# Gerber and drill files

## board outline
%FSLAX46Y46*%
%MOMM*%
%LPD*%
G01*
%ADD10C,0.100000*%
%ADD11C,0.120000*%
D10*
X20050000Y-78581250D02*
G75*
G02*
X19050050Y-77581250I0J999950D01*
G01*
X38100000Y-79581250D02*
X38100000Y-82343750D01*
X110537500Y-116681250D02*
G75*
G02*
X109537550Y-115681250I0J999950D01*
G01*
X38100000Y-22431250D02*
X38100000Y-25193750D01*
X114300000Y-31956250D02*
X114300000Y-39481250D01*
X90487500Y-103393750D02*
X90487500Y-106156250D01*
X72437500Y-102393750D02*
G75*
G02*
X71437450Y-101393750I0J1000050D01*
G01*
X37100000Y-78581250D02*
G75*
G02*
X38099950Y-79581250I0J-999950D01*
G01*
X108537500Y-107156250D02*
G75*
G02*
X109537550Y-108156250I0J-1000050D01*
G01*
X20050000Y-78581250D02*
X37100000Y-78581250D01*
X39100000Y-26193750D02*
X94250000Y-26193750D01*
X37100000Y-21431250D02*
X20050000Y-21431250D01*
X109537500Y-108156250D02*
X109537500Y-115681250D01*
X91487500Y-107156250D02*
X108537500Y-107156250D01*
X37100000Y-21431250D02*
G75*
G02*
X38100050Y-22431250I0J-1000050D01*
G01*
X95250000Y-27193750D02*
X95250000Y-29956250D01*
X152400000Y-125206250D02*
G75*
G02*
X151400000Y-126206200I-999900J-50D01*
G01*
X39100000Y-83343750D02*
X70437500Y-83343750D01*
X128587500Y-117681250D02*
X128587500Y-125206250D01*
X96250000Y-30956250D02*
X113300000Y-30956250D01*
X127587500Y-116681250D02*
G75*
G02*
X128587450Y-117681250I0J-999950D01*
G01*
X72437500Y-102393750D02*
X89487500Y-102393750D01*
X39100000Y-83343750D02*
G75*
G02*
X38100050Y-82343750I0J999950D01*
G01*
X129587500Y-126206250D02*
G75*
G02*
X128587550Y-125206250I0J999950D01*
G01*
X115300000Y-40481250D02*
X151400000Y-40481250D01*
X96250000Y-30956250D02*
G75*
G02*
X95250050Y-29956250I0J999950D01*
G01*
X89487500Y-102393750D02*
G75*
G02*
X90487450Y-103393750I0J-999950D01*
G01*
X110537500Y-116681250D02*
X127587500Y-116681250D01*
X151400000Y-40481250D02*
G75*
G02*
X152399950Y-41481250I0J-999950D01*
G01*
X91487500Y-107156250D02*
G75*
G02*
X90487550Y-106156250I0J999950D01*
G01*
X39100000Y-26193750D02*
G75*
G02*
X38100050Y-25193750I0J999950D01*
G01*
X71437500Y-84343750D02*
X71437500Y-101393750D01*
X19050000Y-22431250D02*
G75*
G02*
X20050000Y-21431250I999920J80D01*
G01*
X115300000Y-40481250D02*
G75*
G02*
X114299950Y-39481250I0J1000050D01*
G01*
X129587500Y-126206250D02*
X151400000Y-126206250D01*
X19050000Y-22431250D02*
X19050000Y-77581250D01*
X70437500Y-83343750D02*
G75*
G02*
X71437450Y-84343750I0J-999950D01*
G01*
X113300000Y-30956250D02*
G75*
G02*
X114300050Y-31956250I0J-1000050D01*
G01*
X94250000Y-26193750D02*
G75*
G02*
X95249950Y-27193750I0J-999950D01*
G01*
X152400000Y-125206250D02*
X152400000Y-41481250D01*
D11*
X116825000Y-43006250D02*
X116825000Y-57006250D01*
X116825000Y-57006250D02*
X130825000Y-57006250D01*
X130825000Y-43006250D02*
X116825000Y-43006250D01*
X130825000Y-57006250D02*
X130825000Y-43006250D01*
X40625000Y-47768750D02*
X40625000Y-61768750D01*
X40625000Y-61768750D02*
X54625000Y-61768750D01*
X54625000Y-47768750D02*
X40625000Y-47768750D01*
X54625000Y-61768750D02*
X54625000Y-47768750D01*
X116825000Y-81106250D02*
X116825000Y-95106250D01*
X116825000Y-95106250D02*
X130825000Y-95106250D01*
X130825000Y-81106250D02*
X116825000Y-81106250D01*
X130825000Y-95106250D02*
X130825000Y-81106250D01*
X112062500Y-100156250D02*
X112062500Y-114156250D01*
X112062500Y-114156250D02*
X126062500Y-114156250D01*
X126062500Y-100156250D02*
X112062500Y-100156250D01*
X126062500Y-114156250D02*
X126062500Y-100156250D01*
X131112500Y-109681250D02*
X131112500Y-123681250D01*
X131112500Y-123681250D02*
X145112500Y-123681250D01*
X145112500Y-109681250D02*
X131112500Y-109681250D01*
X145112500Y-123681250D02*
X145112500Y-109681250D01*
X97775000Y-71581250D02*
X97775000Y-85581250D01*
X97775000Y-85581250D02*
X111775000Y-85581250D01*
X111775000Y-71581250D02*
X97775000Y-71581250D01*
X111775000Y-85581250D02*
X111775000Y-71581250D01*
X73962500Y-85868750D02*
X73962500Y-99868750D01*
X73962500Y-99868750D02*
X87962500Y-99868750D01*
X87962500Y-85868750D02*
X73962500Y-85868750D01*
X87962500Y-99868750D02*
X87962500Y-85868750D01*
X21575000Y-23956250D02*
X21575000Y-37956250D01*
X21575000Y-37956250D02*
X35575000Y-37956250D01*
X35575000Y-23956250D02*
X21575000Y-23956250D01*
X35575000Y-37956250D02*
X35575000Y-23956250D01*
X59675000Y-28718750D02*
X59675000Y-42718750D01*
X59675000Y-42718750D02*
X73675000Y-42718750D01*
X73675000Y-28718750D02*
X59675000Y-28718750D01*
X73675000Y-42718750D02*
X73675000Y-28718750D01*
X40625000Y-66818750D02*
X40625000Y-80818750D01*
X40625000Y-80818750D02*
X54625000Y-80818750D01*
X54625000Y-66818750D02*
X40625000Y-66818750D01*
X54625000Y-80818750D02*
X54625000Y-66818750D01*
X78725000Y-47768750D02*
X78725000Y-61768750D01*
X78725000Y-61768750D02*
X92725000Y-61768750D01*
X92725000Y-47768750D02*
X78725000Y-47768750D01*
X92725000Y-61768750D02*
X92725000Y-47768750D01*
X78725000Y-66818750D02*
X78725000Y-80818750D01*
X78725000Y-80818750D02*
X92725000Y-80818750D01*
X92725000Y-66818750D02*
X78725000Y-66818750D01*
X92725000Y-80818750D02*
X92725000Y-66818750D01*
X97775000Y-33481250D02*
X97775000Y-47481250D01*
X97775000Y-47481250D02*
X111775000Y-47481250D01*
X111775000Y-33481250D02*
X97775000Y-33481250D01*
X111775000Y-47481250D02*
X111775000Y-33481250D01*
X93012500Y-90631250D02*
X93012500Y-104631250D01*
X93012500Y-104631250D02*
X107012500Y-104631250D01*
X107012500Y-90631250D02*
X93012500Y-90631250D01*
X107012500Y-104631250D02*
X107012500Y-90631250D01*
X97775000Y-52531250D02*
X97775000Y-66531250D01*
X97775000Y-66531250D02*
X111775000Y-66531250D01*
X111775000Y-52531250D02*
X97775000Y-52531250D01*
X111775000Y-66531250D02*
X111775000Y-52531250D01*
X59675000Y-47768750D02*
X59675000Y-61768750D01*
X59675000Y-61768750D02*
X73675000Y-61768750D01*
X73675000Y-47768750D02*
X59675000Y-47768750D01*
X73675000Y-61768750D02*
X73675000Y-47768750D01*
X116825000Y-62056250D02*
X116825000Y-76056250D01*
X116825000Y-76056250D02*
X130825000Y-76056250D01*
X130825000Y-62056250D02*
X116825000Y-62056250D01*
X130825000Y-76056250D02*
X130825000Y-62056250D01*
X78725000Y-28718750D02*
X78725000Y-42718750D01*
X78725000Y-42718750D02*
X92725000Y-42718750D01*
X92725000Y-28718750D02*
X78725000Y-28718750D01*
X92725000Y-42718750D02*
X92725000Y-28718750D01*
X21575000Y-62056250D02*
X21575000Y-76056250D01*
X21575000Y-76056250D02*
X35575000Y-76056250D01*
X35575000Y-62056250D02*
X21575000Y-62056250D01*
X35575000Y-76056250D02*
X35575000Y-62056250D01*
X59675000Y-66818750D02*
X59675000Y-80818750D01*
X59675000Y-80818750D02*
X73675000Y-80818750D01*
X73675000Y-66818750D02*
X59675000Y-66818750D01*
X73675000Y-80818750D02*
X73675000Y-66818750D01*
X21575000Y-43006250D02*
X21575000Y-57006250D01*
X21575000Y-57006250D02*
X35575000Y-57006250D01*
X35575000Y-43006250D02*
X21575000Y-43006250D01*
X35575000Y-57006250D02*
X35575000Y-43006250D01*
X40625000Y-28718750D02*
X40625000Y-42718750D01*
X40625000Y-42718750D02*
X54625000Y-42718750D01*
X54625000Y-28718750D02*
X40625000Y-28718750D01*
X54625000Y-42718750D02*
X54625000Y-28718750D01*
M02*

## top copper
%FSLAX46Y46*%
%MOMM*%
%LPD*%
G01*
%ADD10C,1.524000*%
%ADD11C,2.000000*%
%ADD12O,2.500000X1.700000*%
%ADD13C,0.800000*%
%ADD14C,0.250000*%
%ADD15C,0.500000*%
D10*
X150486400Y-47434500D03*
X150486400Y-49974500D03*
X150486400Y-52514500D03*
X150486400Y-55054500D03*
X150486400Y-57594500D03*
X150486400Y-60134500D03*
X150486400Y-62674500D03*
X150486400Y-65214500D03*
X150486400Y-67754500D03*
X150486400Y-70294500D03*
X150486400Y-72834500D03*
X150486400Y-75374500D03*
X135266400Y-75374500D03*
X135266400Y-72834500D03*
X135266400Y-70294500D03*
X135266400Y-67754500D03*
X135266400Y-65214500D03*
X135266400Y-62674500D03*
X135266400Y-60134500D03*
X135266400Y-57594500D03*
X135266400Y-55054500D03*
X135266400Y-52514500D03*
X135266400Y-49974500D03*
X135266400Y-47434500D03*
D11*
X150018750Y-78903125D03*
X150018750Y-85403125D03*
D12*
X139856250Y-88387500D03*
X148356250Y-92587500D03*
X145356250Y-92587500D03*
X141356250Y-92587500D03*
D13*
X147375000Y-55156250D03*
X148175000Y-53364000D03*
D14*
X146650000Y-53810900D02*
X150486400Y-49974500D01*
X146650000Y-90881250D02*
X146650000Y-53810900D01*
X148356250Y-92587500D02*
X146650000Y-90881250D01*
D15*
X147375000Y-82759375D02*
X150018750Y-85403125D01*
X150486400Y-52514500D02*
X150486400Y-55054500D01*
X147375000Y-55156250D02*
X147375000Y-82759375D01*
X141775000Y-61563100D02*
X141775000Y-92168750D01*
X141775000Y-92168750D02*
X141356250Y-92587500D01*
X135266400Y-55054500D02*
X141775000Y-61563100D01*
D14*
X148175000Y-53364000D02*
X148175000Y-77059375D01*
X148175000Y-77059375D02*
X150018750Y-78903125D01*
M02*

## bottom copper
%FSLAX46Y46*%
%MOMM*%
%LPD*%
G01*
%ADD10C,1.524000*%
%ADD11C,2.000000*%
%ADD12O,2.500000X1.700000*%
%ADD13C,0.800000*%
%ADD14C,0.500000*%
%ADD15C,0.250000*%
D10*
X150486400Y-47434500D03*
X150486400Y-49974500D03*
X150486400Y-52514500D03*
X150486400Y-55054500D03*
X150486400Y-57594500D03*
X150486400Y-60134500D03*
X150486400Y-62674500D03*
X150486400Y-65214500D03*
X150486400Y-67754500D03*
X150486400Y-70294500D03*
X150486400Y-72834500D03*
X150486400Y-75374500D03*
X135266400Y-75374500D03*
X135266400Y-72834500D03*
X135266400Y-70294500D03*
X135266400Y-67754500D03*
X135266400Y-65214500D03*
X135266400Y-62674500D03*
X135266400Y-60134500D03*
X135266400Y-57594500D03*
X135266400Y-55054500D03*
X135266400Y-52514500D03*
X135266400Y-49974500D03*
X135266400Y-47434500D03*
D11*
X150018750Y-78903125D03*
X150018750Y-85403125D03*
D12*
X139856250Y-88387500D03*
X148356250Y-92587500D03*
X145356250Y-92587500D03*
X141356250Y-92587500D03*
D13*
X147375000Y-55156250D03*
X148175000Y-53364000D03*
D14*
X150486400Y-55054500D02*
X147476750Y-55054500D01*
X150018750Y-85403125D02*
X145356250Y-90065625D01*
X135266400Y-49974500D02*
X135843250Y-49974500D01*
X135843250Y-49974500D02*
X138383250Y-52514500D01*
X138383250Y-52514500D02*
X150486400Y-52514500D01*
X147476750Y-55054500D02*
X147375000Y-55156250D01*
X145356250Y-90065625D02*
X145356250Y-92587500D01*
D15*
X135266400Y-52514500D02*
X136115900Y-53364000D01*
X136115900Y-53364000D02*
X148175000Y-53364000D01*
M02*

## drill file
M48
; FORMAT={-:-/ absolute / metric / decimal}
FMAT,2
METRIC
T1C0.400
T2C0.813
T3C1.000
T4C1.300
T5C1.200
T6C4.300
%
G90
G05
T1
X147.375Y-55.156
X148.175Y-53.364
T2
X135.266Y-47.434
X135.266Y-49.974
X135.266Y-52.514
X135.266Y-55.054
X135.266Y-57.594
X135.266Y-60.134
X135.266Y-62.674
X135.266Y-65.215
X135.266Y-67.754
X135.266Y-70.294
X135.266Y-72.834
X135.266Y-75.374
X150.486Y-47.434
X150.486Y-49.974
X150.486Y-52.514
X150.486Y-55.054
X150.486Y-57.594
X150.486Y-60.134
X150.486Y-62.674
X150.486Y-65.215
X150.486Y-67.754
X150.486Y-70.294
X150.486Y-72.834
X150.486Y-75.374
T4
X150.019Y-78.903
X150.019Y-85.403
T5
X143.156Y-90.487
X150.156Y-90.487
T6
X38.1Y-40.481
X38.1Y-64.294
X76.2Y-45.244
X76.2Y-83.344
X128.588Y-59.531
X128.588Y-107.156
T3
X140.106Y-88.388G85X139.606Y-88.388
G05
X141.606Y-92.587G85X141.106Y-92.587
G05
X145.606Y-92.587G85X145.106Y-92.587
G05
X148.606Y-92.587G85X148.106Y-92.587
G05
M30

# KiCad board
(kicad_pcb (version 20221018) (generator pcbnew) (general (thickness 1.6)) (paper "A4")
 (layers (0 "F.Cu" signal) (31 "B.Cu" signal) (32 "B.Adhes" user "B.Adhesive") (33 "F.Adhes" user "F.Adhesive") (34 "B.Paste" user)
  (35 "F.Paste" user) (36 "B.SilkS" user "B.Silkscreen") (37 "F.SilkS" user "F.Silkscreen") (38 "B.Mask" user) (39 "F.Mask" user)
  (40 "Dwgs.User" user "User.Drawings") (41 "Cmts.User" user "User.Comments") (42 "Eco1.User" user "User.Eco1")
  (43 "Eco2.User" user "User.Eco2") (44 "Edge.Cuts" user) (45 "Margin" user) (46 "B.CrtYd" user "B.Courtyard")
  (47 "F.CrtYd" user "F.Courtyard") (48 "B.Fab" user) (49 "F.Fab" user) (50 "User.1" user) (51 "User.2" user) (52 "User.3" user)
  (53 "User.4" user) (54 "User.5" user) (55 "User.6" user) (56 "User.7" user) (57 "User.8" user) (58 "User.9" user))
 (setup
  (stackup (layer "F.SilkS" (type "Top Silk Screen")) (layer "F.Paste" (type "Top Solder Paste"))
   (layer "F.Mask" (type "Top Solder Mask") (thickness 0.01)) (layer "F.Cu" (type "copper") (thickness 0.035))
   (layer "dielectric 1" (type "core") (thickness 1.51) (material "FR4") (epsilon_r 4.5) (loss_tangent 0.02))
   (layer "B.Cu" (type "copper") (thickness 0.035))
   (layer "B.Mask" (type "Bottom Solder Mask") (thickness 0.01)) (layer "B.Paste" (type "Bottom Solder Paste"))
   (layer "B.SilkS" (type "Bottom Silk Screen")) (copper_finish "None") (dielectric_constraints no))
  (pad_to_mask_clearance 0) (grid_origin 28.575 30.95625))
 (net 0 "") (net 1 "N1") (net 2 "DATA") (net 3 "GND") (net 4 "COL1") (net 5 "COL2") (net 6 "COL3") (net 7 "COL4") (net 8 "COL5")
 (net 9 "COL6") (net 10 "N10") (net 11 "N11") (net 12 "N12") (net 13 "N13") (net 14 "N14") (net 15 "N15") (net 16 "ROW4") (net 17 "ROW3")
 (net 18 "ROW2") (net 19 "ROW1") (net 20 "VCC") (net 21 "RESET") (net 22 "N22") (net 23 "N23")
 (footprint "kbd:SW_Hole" (layer "F.Cu") (at 123.825 50.00625)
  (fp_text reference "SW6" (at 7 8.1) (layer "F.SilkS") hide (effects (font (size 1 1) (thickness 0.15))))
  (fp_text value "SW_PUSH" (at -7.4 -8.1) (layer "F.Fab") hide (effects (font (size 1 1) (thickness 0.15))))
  (fp_line (start -7 -7) (end -7 7) (stroke (width 0.12) (type solid)) (layer "Edge.Cuts"))
  (fp_line (start -7 7) (end 7 7) (stroke (width 0.12) (type solid)) (layer "Edge.Cuts"))
  (fp_line (start 7 -7) (end -7 -7) (stroke (width 0.12) (type solid)) (layer "Edge.Cuts"))
  (fp_line (start 7 7) (end 7 -7) (stroke (width 0.12) (type solid)) (layer "Edge.Cuts")))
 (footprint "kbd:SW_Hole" (layer "F.Cu") (at 47.625 54.76875)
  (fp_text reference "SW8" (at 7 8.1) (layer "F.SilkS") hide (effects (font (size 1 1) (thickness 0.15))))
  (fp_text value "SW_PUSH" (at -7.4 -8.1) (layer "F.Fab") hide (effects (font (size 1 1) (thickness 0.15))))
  (fp_line (start -7 -7) (end -7 7) (stroke (width 0.12) (type solid)) (layer "Edge.Cuts"))
  (fp_line (start -7 7) (end 7 7) (stroke (width 0.12) (type solid)) (layer "Edge.Cuts"))
  (fp_line (start 7 -7) (end -7 -7) (stroke (width 0.12) (type solid)) (layer "Edge.Cuts"))
  (fp_line (start 7 7) (end 7 -7) (stroke (width 0.12) (type solid)) (layer "Edge.Cuts")))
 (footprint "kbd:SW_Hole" (layer "F.Cu") (at 123.825 88.10625)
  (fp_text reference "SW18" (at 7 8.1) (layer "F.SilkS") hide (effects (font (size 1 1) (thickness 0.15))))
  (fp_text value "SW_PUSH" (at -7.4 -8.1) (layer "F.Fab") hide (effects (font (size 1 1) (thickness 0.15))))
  (fp_line (start -7 -7) (end -7 7) (stroke (width 0.12) (type solid)) (layer "Edge.Cuts"))
  (fp_line (start -7 7) (end 7 7) (stroke (width 0.12) (type solid)) (layer "Edge.Cuts"))
  (fp_line (start 7 -7) (end -7 -7) (stroke (width 0.12) (type solid)) (layer "Edge.Cuts"))
  (fp_line (start 7 7) (end 7 -7) (stroke (width 0.12) (type solid)) (layer "Edge.Cuts")))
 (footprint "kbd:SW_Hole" (layer "F.Cu") (at 119.0625 107.15625)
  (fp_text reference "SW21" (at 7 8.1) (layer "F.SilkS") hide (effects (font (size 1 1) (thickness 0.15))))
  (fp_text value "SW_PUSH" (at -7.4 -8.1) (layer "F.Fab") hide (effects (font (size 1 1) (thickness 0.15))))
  (fp_line (start -7 -7) (end -7 7) (stroke (width 0.12) (type solid)) (layer "Edge.Cuts"))
  (fp_line (start -7 7) (end 7 7) (stroke (width 0.12) (type solid)) (layer "Edge.Cuts"))
  (fp_line (start 7 -7) (end -7 -7) (stroke (width 0.12) (type solid)) (layer "Edge.Cuts"))
  (fp_line (start 7 7) (end 7 -7) (stroke (width 0.12) (type solid)) (layer "Edge.Cuts")))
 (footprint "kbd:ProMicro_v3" (layer "F.Cu") (at 142.875 61.9125)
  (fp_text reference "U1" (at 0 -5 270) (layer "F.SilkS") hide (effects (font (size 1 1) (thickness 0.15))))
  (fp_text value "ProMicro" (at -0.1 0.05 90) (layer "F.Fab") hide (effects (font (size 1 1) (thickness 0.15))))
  (pad "1" thru_hole circle (at 7.6114 -14.478) (size 1.524 1.524) (drill 0.8128) (layers "*.Cu" "B.Mask") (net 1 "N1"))
  (pad "2" thru_hole circle (at 7.6114 -11.938) (size 1.524 1.524) (drill 0.8128) (layers "*.Cu" "B.Mask") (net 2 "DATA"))
  (pad "3" thru_hole circle (at 7.6114 -9.398) (size 1.524 1.524) (drill 0.8128) (layers "*.Cu" "B.Mask") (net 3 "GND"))
  (pad "4" thru_hole circle (at 7.6114 -6.858) (size 1.524 1.524) (drill 0.8128) (layers "*.Cu" "B.Mask") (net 3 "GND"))
  (pad "5" thru_hole circle (at 7.6114 -4.318) (size 1.524 1.524) (drill 0.8128) (layers "*.Cu" "B.Mask") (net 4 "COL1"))
  (pad "6" thru_hole circle (at 7.6114 -1.778) (size 1.524 1.524) (drill 0.8128) (layers "*.Cu" "B.Mask") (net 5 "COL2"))
  (pad "7" thru_hole circle (at 7.6114 0.762) (size 1.524 1.524) (drill 0.8128) (layers "*.Cu" "B.Mask") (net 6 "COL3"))
  (pad "8" thru_hole circle (at 7.6114 3.302) (size 1.524 1.524) (drill 0.8128) (layers "*.Cu" "B.Mask") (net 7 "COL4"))
  (pad "9" thru_hole circle (at 7.6114 5.842) (size 1.524 1.524) (drill 0.8128) (layers "*.Cu" "B.Mask") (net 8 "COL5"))
  (pad "10" thru_hole circle (at 7.6114 8.382) (size 1.524 1.524) (drill 0.8128) (layers "*.Cu" "B.Mask") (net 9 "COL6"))
  (pad "11" thru_hole circle (at 7.6114 10.922) (size 1.524 1.524) (drill 0.8128) (layers "*.Cu" "B.Mask") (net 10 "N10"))
  (pad "12" thru_hole circle (at 7.6114 13.462) (size 1.524 1.524) (drill 0.8128) (layers "*.Cu" "B.Mask") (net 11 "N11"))
  (pad "13" thru_hole circle (at -7.6086 13.462) (size 1.524 1.524) (drill 0.8128) (layers "*.Cu" "B.Mask") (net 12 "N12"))
  (pad "14" thru_hole circle (at -7.6086 10.922) (size 1.524 1.524) (drill 0.8128) (layers "*.Cu" "B.Mask") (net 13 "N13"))
  (pad "15" thru_hole circle (at -7.6086 8.382) (size 1.524 1.524) (drill 0.8128) (layers "*.Cu" "B.Mask") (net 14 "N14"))
  (pad "16" thru_hole circle (at -7.6086 5.842) (size 1.524 1.524) (drill 0.8128) (layers "*.Cu" "B.Mask") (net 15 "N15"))
  (pad "17" thru_hole circle (at -7.6086 3.302) (size 1.524 1.524) (drill 0.8128) (layers "*.Cu" "B.Mask") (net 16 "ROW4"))
  (pad "18" thru_hole circle (at -7.6086 0.762) (size 1.524 1.524) (drill 0.8128) (layers "*.Cu" "B.Mask") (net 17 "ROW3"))
  (pad "19" thru_hole circle (at -7.6086 -1.778) (size 1.524 1.524) (drill 0.8128) (layers "*.Cu" "B.Mask") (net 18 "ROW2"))
  (pad "20" thru_hole circle (at -7.6086 -4.318) (size 1.524 1.524) (drill 0.8128) (layers "*.Cu" "B.Mask") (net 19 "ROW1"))
  (pad "21" thru_hole circle (at -7.6086 -6.858) (size 1.524 1.524) (drill 0.8128) (layers "*.Cu" "B.Mask") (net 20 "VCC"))
  (pad "22" thru_hole circle (at -7.6086 -9.398) (size 1.524 1.524) (drill 0.8128) (layers "*.Cu" "B.Mask") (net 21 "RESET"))
  (pad "23" thru_hole circle (at -7.6086 -11.938) (size 1.524 1.524) (drill 0.8128) (layers "*.Cu" "B.Mask") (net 3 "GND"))
  (pad "24" thru_hole circle (at -7.6086 -14.478) (size 1.524 1.524) (drill 0.8128) (layers "*.Cu" "B.Mask") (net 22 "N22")))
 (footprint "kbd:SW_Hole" (layer "F.Cu") (at 138.1125 116.68125)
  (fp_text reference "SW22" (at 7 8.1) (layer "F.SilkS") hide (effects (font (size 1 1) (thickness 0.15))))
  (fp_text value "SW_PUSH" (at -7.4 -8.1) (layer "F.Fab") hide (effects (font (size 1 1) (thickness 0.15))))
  (fp_line (start -7 -7) (end -7 7) (stroke (width 0.12) (type solid)) (layer "Edge.Cuts"))
  (fp_line (start -7 7) (end 7 7) (stroke (width 0.12) (type solid)) (layer "Edge.Cuts"))
  (fp_line (start 7 -7) (end -7 -7) (stroke (width 0.12) (type solid)) (layer "Edge.Cuts"))
  (fp_line (start 7 7) (end 7 -7) (stroke (width 0.12) (type solid)) (layer "Edge.Cuts")))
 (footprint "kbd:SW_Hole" (layer "F.Cu") (at 104.775 78.58125)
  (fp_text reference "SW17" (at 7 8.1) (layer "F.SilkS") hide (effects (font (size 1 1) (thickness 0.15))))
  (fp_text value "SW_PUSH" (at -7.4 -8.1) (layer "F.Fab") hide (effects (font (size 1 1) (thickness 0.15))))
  (fp_line (start -7 -7) (end -7 7) (stroke (width 0.12) (type solid)) (layer "Edge.Cuts"))
  (fp_line (start -7 7) (end 7 7) (stroke (width 0.12) (type solid)) (layer "Edge.Cuts"))
  (fp_line (start 7 -7) (end -7 -7) (stroke (width 0.12) (type solid)) (layer "Edge.Cuts"))
  (fp_line (start 7 7) (end 7 -7) (stroke (width 0.12) (type solid)) (layer "Edge.Cuts")))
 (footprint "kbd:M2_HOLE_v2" (layer "F.Cu") (at 76.2 45.24375)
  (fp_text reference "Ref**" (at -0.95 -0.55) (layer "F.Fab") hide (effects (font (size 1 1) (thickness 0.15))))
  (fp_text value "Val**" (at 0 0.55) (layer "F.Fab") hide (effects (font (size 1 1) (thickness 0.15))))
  (pad "" np_thru_hole circle (at 0 0) (size 4.3 4.3) (drill 4.3) (layers "*.Cu" "*.Mask")))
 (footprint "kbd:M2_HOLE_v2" (layer "F.Cu") (at 128.5875 59.53125)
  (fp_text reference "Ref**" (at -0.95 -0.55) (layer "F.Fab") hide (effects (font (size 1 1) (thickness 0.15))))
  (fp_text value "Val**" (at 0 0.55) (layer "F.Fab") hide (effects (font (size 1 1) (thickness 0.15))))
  (pad "" np_thru_hole circle (at 0 0) (size 4.3 4.3) (drill 4.3) (layers "*.Cu" "*.Mask")))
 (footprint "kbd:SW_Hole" (layer "F.Cu") (at 80.9625 92.86875)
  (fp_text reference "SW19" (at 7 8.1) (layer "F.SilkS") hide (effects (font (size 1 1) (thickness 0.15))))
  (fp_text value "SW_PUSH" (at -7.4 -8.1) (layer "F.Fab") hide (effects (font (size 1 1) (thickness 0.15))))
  (fp_line (start -7 -7) (end -7 7) (stroke (width 0.12) (type solid)) (layer "Edge.Cuts"))
  (fp_line (start -7 7) (end 7 7) (stroke (width 0.12) (type solid)) (layer "Edge.Cuts"))
  (fp_line (start 7 -7) (end -7 -7) (stroke (width 0.12) (type solid)) (layer "Edge.Cuts"))
  (fp_line (start 7 7) (end 7 -7) (stroke (width 0.12) (type solid)) (layer "Edge.Cuts")))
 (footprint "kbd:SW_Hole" (layer "F.Cu") (at 28.575 30.95625)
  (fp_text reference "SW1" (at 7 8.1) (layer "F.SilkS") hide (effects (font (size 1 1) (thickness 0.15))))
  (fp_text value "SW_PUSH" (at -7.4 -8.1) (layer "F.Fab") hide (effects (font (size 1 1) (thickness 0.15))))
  (fp_line (start -7 -7) (end -7 7) (stroke (width 0.12) (type solid)) (layer "Edge.Cuts"))
  (fp_line (start -7 7) (end 7 7) (stroke (width 0.12) (type solid)) (layer "Edge.Cuts"))
  (fp_line (start 7 -7) (end -7 -7) (stroke (width 0.12) (type solid)) (layer "Edge.Cuts"))
  (fp_line (start 7 7) (end 7 -7) (stroke (width 0.12) (type solid)) (layer "Edge.Cuts")))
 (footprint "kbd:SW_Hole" (layer "F.Cu") (at 66.675 35.71875)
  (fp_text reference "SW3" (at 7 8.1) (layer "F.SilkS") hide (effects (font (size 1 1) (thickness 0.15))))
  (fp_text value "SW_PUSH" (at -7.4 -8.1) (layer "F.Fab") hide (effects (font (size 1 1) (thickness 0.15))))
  (fp_line (start -7 -7) (end -7 7) (stroke (width 0.12) (type solid)) (layer "Edge.Cuts"))
  (fp_line (start -7 7) (end 7 7) (stroke (width 0.12) (type solid)) (layer "Edge.Cuts"))
  (fp_line (start 7 -7) (end -7 -7) (stroke (width 0.12) (type solid)) (layer "Edge.Cuts"))
  (fp_line (start 7 7) (end 7 -7) (stroke (width 0.12) (type solid)) (layer "Edge.Cuts")))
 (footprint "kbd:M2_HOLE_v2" (layer "F.Cu") (at 38.1 64.29375)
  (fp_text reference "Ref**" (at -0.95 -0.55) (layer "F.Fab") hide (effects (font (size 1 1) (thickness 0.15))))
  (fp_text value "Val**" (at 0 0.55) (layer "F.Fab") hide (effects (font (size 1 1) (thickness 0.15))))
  (pad "" np_thru_hole circle (at 0 0) (size 4.3 4.3) (drill 4.3) (layers "*.Cu" "*.Mask")))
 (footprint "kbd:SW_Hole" (layer "F.Cu") (at 47.625 73.81875)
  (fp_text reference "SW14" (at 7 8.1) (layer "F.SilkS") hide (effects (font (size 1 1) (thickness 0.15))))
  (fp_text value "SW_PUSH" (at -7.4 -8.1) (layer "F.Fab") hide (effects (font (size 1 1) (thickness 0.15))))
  (fp_line (start -7 -7) (end -7 7) (stroke (width 0.12) (type solid)) (layer "Edge.Cuts"))
  (fp_line (start -7 7) (end 7 7) (stroke (width 0.12) (type solid)) (layer "Edge.Cuts"))
  (fp_line (start 7 -7) (end -7 -7) (stroke (width 0.12) (type solid)) (layer "Edge.Cuts"))
  (fp_line (start 7 7) (end 7 -7) (stroke (width 0.12) (type solid)) (layer "Edge.Cuts")))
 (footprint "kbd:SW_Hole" (layer "F.Cu") (at 85.725 54.76875)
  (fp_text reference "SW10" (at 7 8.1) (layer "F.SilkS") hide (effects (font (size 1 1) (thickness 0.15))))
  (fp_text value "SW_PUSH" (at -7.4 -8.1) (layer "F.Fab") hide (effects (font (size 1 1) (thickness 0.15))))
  (fp_line (start -7 -7) (end -7 7) (stroke (width 0.12) (type solid)) (layer "Edge.Cuts"))
  (fp_line (start -7 7) (end 7 7) (stroke (width 0.12) (type solid)) (layer "Edge.Cuts"))
  (fp_line (start 7 -7) (end -7 -7) (stroke (width 0.12) (type solid)) (layer "Edge.Cuts"))
  (fp_line (start 7 7) (end 7 -7) (stroke (width 0.12) (type solid)) (layer "Edge.Cuts")))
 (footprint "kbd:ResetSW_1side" (layer "F.Cu") (at 150.01875 82.153125 90)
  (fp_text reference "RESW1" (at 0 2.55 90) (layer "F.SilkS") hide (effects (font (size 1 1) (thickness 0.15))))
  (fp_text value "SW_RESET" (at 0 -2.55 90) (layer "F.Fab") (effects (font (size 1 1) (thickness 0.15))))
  (pad "1" thru_hole circle (at 3.25 0 90) (size 2 2) (drill 1.3) (layers "*.Cu" "B.Mask") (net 21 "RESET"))
  (pad "2" thru_hole circle (at -3.25 0 90) (size 2 2) (drill 1.3) (layers "*.Cu" "B.Mask") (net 3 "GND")))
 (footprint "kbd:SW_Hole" (layer "F.Cu") (at 85.725 73.81875)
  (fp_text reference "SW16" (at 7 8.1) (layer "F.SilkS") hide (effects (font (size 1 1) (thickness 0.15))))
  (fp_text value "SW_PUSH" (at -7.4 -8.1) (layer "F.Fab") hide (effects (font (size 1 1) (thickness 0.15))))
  (fp_line (start -7 -7) (end -7 7) (stroke (width 0.12) (type solid)) (layer "Edge.Cuts"))
  (fp_line (start -7 7) (end 7 7) (stroke (width 0.12) (type solid)) (layer "Edge.Cuts"))
  (fp_line (start 7 -7) (end -7 -7) (stroke (width 0.12) (type solid)) (layer "Edge.Cuts"))
  (fp_line (start 7 7) (end 7 -7) (stroke (width 0.12) (type solid)) (layer "Edge.Cuts")))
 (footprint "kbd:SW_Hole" (layer "F.Cu") (at 104.775 40.48125)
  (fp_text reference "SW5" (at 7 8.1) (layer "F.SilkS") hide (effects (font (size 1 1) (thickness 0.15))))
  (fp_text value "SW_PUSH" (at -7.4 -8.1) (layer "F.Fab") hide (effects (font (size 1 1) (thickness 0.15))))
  (fp_line (start -7 -7) (end -7 7) (stroke (width 0.12) (type solid)) (layer "Edge.Cuts"))
  (fp_line (start -7 7) (end 7 7) (stroke (width 0.12) (type solid)) (layer "Edge.Cuts"))
  (fp_line (start 7 -7) (end -7 -7) (stroke (width 0.12) (type solid)) (layer "Edge.Cuts"))
  (fp_line (start 7 7) (end 7 -7) (stroke (width 0.12) (type solid)) (layer "Edge.Cuts")))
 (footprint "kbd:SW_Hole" (layer "F.Cu") (at 100.0125 97.63125)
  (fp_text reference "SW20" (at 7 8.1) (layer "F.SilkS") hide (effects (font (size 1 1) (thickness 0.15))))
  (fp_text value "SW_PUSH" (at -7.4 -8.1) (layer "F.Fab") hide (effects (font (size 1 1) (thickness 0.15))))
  (fp_line (start -7 -7) (end -7 7) (stroke (width 0.12) (type solid)) (layer "Edge.Cuts"))
  (fp_line (start -7 7) (end 7 7) (stroke (width 0.12) (type solid)) (layer "Edge.Cuts"))
  (fp_line (start 7 -7) (end -7 -7) (stroke (width 0.12) (type solid)) (layer "Edge.Cuts"))
  (fp_line (start 7 7) (end 7 -7) (stroke (width 0.12) (type solid)) (layer "Edge.Cuts")))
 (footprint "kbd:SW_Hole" (layer "F.Cu") (at 104.775 59.53125)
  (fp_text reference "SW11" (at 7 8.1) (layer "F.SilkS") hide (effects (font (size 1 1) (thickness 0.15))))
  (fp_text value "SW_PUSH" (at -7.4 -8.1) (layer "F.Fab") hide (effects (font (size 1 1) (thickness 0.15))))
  (fp_line (start -7 -7) (end -7 7) (stroke (width 0.12) (type solid)) (layer "Edge.Cuts"))
  (fp_line (start -7 7) (end 7 7) (stroke (width 0.12) (type solid)) (layer "Edge.Cuts"))
  (fp_line (start 7 -7) (end -7 -7) (stroke (width 0.12) (type solid)) (layer "Edge.Cuts"))
  (fp_line (start 7 7) (end 7 -7) (stroke (width 0.12) (type solid)) (layer "Edge.Cuts")))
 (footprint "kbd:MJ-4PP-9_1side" (layer "F.Cu") (at 151.65625 90.4875 -90)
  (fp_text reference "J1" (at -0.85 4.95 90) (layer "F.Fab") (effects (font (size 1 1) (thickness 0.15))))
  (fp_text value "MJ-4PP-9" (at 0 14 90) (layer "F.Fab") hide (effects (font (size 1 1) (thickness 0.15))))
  (pad "" np_thru_hole circle (at 0 1.5 270) (size 1.2 1.2) (drill 1.2) (layers "*.Cu" "*.Mask"))
  (pad "" np_thru_hole circle (at 0 8.5 270) (size 1.2 1.2) (drill 1.2) (layers "*.Cu" "*.Mask"))
  (pad "A" thru_hole oval (at -2.1 11.8 270) (size 1.7 2.5) (drill oval 1 1.5) (layers "*.Cu" "B.Mask") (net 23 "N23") (clearance 0.15))
  (pad "B" thru_hole oval (at 2.1 3.3 270) (size 1.7 2.5) (drill oval 1 1.5) (layers "*.Cu" "B.Mask") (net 2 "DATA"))
  (pad "C" thru_hole oval (at 2.1 6.3 270) (size 1.7 2.5) (drill oval 1 1.5) (layers "*.Cu" "B.Mask") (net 3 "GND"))
  (pad "D" thru_hole oval (at 2.1 10.3 270) (size 1.7 2.5) (drill oval 1 1.5) (layers "*.Cu" "B.Mask") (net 20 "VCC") (clearance 0.15)))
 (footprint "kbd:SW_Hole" (layer "F.Cu") (at 66.675 54.76875)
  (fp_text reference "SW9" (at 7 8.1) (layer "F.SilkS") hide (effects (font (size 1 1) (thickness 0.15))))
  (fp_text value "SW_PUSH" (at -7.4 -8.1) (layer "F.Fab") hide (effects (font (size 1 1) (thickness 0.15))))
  (fp_line (start -7 -7) (end -7 7) (stroke (width 0.12) (type solid)) (layer "Edge.Cuts"))
  (fp_line (start -7 7) (end 7 7) (stroke (width 0.12) (type solid)) (layer "Edge.Cuts"))
  (fp_line (start 7 -7) (end -7 -7) (stroke (width 0.12) (type solid)) (layer "Edge.Cuts"))
  (fp_line (start 7 7) (end 7 -7) (stroke (width 0.12) (type solid)) (layer "Edge.Cuts")))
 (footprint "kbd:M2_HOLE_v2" (layer "F.Cu") (at 38.1 40.48125)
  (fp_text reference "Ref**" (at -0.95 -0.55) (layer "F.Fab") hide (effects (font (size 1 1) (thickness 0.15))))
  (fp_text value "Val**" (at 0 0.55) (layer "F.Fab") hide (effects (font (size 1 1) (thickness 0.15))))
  (pad "" np_thru_hole circle (at 0 0) (size 4.3 4.3) (drill 4.3) (layers "*.Cu" "*.Mask")))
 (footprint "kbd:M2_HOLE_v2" (layer "F.Cu") (at 128.5875 107.15625)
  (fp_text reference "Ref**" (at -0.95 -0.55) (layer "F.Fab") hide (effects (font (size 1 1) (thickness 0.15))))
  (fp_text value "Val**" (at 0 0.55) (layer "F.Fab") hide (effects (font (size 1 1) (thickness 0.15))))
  (pad "" np_thru_hole circle (at 0 0) (size 4.3 4.3) (drill 4.3) (layers "*.Cu" "*.Mask")))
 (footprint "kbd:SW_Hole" (layer "F.Cu") (at 123.825 69.05625)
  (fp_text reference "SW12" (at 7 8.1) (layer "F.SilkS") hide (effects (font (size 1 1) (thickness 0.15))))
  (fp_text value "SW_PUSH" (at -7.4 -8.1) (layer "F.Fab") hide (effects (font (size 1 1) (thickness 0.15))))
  (fp_line (start -7 -7) (end -7 7) (stroke (width 0.12) (type solid)) (layer "Edge.Cuts"))
  (fp_line (start -7 7) (end 7 7) (stroke (width 0.12) (type solid)) (layer "Edge.Cuts"))
  (fp_line (start 7 -7) (end -7 -7) (stroke (width 0.12) (type solid)) (layer "Edge.Cuts"))
  (fp_line (start 7 7) (end 7 -7) (stroke (width 0.12) (type solid)) (layer "Edge.Cuts")))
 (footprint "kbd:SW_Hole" (layer "F.Cu") (at 85.725 35.71875)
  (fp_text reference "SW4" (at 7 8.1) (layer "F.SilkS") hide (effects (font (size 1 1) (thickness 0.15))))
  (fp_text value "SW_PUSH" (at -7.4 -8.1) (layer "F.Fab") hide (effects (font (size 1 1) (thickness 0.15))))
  (fp_line (start -7 -7) (end -7 7) (stroke (width 0.12) (type solid)) (layer "Edge.Cuts"))
  (fp_line (start -7 7) (end 7 7) (stroke (width 0.12) (type solid)) (layer "Edge.Cuts"))
  (fp_line (start 7 -7) (end -7 -7) (stroke (width 0.12) (type solid)) (layer "Edge.Cuts"))
  (fp_line (start 7 7) (end 7 -7) (stroke (width 0.12) (type solid)) (layer "Edge.Cuts")))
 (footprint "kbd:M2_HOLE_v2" (layer "F.Cu") (at 76.2 83.34375)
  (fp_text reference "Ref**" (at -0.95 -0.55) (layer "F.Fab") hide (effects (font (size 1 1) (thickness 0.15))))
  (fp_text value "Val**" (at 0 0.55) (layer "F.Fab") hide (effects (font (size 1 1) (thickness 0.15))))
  (pad "" np_thru_hole circle (at 0 0) (size 4.3 4.3) (drill 4.3) (layers "*.Cu" "*.Mask")))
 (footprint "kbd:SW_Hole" (layer "F.Cu") (at 28.575 69.05625)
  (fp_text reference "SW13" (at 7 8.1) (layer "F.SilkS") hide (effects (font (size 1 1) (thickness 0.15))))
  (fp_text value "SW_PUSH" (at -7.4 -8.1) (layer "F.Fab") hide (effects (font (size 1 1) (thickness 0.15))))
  (fp_line (start -7 -7) (end -7 7) (stroke (width 0.12) (type solid)) (layer "Edge.Cuts"))
  (fp_line (start -7 7) (end 7 7) (stroke (width 0.12) (type solid)) (layer "Edge.Cuts"))
  (fp_line (start 7 -7) (end -7 -7) (stroke (width 0.12) (type solid)) (layer "Edge.Cuts"))
  (fp_line (start 7 7) (end 7 -7) (stroke (width 0.12) (type solid)) (layer "Edge.Cuts")))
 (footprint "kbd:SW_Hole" (layer "F.Cu") (at 66.675 73.81875)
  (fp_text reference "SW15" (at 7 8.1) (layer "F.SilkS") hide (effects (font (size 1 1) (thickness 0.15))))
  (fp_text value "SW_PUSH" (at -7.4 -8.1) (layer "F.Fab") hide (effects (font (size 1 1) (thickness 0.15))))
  (fp_line (start -7 -7) (end -7 7) (stroke (width 0.12) (type solid)) (layer "Edge.Cuts"))
  (fp_line (start -7 7) (end 7 7) (stroke (width 0.12) (type solid)) (layer "Edge.Cuts"))
  (fp_line (start 7 -7) (end -7 -7) (stroke (width 0.12) (type solid)) (layer "Edge.Cuts"))
  (fp_line (start 7 7) (end 7 -7) (stroke (width 0.12) (type solid)) (layer "Edge.Cuts")))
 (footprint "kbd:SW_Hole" (layer "F.Cu") (at 28.575 50.00625)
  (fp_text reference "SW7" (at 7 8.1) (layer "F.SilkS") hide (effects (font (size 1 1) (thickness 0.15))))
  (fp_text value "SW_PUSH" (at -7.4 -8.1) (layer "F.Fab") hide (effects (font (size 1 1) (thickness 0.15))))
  (fp_line (start -7 -7) (end -7 7) (stroke (width 0.12) (type solid)) (layer "Edge.Cuts"))
  (fp_line (start -7 7) (end 7 7) (stroke (width 0.12) (type solid)) (layer "Edge.Cuts"))
  (fp_line (start 7 -7) (end -7 -7) (stroke (width 0.12) (type solid)) (layer "Edge.Cuts"))
  (fp_line (start 7 7) (end 7 -7) (stroke (width 0.12) (type solid)) (layer "Edge.Cuts")))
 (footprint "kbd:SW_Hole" (layer "F.Cu") (at 47.625 35.71875)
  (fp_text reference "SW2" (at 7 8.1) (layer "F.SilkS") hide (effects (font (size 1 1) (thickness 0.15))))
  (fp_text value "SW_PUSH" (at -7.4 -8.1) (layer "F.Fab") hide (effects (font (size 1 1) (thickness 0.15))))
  (fp_line (start -7 -7) (end -7 7) (stroke (width 0.12) (type solid)) (layer "Edge.Cuts"))
  (fp_line (start -7 7) (end 7 7) (stroke (width 0.12) (type solid)) (layer "Edge.Cuts"))
  (fp_line (start 7 -7) (end -7 -7) (stroke (width 0.12) (type solid)) (layer "Edge.Cuts"))
  (fp_line (start 7 7) (end 7 -7) (stroke (width 0.12) (type solid)) (layer "Edge.Cuts")))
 (gr_arc (start 20.05 78.58125) (mid 19.342893 78.288357) (end 19.05 77.58125) (stroke (width 0.1) (type default)) (layer "Edge.Cuts"))
 (gr_line (start 38.1 79.58125) (end 38.1 82.34375) (stroke (width 0.1) (type default)) (layer "Edge.Cuts"))
 (gr_arc (start 110.5375 116.68125) (mid 109.830393 116.388357) (end 109.5375 115.68125) (stroke (width 0.1) (type default))
  (layer "Edge.Cuts"))
 (gr_line (start 38.1 22.43125) (end 38.1 25.19375) (stroke (width 0.1) (type default)) (layer "Edge.Cuts"))
 (gr_line (start 114.3 31.95625) (end 114.3 39.48125) (stroke (width 0.1) (type default)) (layer "Edge.Cuts"))
 (gr_line (start 90.4875 103.39375) (end 90.4875 106.15625) (stroke (width 0.1) (type default)) (layer "Edge.Cuts"))
 (gr_arc (start 72.4375 102.39375) (mid 71.730411 102.100854) (end 71.4375 101.39375) (stroke (width 0.1) (type default))
  (layer "Edge.Cuts"))
 (gr_arc (start 37.1 78.58125) (mid 37.807107 78.874143) (end 38.1 79.58125) (stroke (width 0.1) (type default)) (layer "Edge.Cuts"))
 (gr_arc (start 108.5375 107.15625) (mid 109.244589 107.449146) (end 109.5375 108.15625) (stroke (width 0.1) (type default))
  (layer "Edge.Cuts"))
 (gr_line (start 20.05 78.58125) (end 37.1 78.58125) (stroke (width 0.1) (type default)) (layer "Edge.Cuts"))
 (gr_line (start 39.1 26.19375) (end 94.25 26.19375) (stroke (width 0.1) (type default)) (layer "Edge.Cuts"))
 (gr_line (start 37.1 21.43125) (end 20.05 21.43125) (stroke (width 0.1) (type default)) (layer "Edge.Cuts"))
 (gr_line (start 109.5375 108.15625) (end 109.5375 115.68125) (stroke (width 0.1) (type default)) (layer "Edge.Cuts"))
 (gr_line (start 91.4875 107.15625) (end 108.5375 107.15625) (stroke (width 0.1) (type default)) (layer "Edge.Cuts"))
 (gr_arc (start 37.1 21.43125) (mid 37.807089 21.724146) (end 38.1 22.43125) (stroke (width 0.1) (type default)) (layer "Edge.Cuts"))
 (gr_line (start 95.25 27.19375) (end 95.25 29.95625) (stroke (width 0.1) (type default)) (layer "Edge.Cuts"))
 (gr_arc (start 152.4 125.20625) (mid 152.107124 125.913389) (end 151.4 126.20625) (stroke (width 0.1) (type default)) (layer "Edge.Cuts"))
 (gr_line (start 39.1 83.34375) (end 70.4375 83.34375) (stroke (width 0.1) (type default)) (layer "Edge.Cuts"))
 (gr_line (start 128.5875 117.68125) (end 128.5875 125.20625) (stroke (width 0.1) (type default)) (layer "Edge.Cuts"))
 (gr_line (start 96.25 30.95625) (end 113.3 30.95625) (stroke (width 0.1) (type default)) (layer "Edge.Cuts"))
 (gr_arc (start 127.5875 116.68125) (mid 128.294607 116.974143) (end 128.5875 117.68125) (stroke (width 0.1) (type default))
  (layer "Edge.Cuts"))
 (gr_line (start 72.4375 102.39375) (end 89.4875 102.39375) (stroke (width 0.1) (type default)) (layer "Edge.Cuts"))
 (gr_arc (start 39.1 83.34375) (mid 38.392893 83.050857) (end 38.1 82.34375) (stroke (width 0.1) (type default)) (layer "Edge.Cuts"))
 (gr_arc (start 129.5875 126.20625) (mid 128.880393 125.913357) (end 128.5875 125.20625) (stroke (width 0.1) (type default))
  (layer "Edge.Cuts"))
 (gr_line (start 115.3 40.48125) (end 151.4 40.48125) (stroke (width 0.1) (type default)) (layer "Edge.Cuts"))
 (gr_arc (start 96.25 30.95625) (mid 95.542893 30.663357) (end 95.25 29.95625) (stroke (width 0.1) (type default)) (layer "Edge.Cuts"))
 (gr_arc (start 89.4875 102.39375) (mid 90.194607 102.686643) (end 90.4875 103.39375) (stroke (width 0.1) (type default))
  (layer "Edge.Cuts"))
 (gr_line (start 110.5375 116.68125) (end 127.5875 116.68125) (stroke (width 0.1) (type default)) (layer "Edge.Cuts"))
 (gr_arc (start 151.4 40.48125) (mid 152.107107 40.774143) (end 152.4 41.48125) (stroke (width 0.1) (type default)) (layer "Edge.Cuts"))
 (gr_arc (start 91.4875 107.15625) (mid 90.780393 106.863357) (end 90.4875 106.15625) (stroke (width 0.1) (type default))
  (layer "Edge.Cuts"))
 (gr_arc (start 39.1 26.19375) (mid 38.392893 25.900857) (end 38.1 25.19375) (stroke (width 0.1) (type default)) (layer "Edge.Cuts"))
 (gr_line (start 71.4375 84.34375) (end 71.4375 101.39375) (stroke (width 0.1) (type default)) (layer "Edge.Cuts"))
 (gr_arc (start 19.05 22.43125) (mid 19.342876 21.724111) (end 20.05 21.43125) (stroke (width 0.1) (type default)) (layer "Edge.Cuts"))
 (gr_arc (start 115.3 40.48125) (mid 114.592911 40.188354) (end 114.3 39.48125) (stroke (width 0.1) (type default)) (layer "Edge.Cuts"))
 (gr_line (start 129.5875 126.20625) (end 151.4 126.20625) (stroke (width 0.1) (type default)) (layer "Edge.Cuts"))
 (gr_line (start 19.05 22.43125) (end 19.05 77.58125) (stroke (width 0.1) (type default)) (layer "Edge.Cuts"))
 (gr_arc (start 70.4375 83.34375) (mid 71.144607 83.636643) (end 71.4375 84.34375) (stroke (width 0.1) (type default)) (layer "Edge.Cuts"))
 (gr_arc (start 113.3 30.95625) (mid 114.007089 31.249146) (end 114.3 31.95625) (stroke (width 0.1) (type default)) (layer "Edge.Cuts"))
 (gr_arc (start 94.25 26.19375) (mid 94.957107 26.486643) (end 95.25 27.19375) (stroke (width 0.1) (type default)) (layer "Edge.Cuts"))
 (gr_line (start 152.4 125.20625) (end 152.4 41.48125) (stroke (width 0.1) (type default)) (layer "Edge.Cuts"))
 (segment (start 146.65 53.8109) (end 150.4864 49.9745) (width 0.25) (layer "F.Cu") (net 2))
 (segment (start 146.65 90.88125) (end 146.65 53.8109) (width 0.25) (layer "F.Cu") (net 2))
 (segment (start 148.35625 92.5875) (end 146.65 90.88125) (width 0.25) (layer "F.Cu") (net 2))
 (segment (start 147.375 82.759375) (end 150.01875 85.403125) (width 0.5) (layer "F.Cu") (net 3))
 (segment (start 150.4864 52.5145) (end 150.4864 55.0545) (width 0.5) (layer "F.Cu") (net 3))
 (segment (start 147.375 55.15625) (end 147.375 82.759375) (width 0.5) (layer "F.Cu") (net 3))
 (via (at 147.375 55.15625) (size 0.8) (drill 0.4) (layers "F.Cu" "B.Cu") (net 3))
 (segment (start 150.4864 55.0545) (end 147.47675 55.0545) (width 0.5) (layer "B.Cu") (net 3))
 (segment (start 150.01875 85.403125) (end 145.35625 90.065625) (width 0.5) (layer "B.Cu") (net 3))
 (segment (start 135.2664 49.9745) (end 135.84325 49.9745) (width 0.5) (layer "B.Cu") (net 3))
 (segment (start 135.84325 49.9745) (end 138.38325 52.5145) (width 0.5) (layer "B.Cu") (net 3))
 (segment (start 138.38325 52.5145) (end 150.4864 52.5145) (width 0.5) (layer "B.Cu") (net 3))
 (segment (start 147.47675 55.0545) (end 147.375 55.15625) (width 0.5) (layer "B.Cu") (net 3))
 (segment (start 145.35625 90.065625) (end 145.35625 92.5875) (width 0.5) (layer "B.Cu") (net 3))
 (segment (start 141.775 61.5631) (end 141.775 92.16875) (width 0.5) (layer "F.Cu") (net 20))
 (segment (start 141.775 92.16875) (end 141.35625 92.5875) (width 0.5) (layer "F.Cu") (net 20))
 (segment (start 135.2664 55.0545) (end 141.775 61.5631) (width 0.5) (layer "F.Cu") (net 20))
 (segment (start 148.175 53.364) (end 148.175 77.059375) (width 0.25) (layer "F.Cu") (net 21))
 (segment (start 148.175 77.059375) (end 150.01875 78.903125) (width 0.25) (layer "F.Cu") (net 21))
 (via (at 148.175 53.364) (size 0.8) (drill 0.4) (layers "F.Cu" "B.Cu") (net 21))
 (segment (start 135.2664 52.5145) (end 136.1159 53.364) (width 0.25) (layer "B.Cu") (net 21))
 (segment (start 136.1159 53.364) (end 148.175 53.364) (width 0.25) (layer "B.Cu") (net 21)))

